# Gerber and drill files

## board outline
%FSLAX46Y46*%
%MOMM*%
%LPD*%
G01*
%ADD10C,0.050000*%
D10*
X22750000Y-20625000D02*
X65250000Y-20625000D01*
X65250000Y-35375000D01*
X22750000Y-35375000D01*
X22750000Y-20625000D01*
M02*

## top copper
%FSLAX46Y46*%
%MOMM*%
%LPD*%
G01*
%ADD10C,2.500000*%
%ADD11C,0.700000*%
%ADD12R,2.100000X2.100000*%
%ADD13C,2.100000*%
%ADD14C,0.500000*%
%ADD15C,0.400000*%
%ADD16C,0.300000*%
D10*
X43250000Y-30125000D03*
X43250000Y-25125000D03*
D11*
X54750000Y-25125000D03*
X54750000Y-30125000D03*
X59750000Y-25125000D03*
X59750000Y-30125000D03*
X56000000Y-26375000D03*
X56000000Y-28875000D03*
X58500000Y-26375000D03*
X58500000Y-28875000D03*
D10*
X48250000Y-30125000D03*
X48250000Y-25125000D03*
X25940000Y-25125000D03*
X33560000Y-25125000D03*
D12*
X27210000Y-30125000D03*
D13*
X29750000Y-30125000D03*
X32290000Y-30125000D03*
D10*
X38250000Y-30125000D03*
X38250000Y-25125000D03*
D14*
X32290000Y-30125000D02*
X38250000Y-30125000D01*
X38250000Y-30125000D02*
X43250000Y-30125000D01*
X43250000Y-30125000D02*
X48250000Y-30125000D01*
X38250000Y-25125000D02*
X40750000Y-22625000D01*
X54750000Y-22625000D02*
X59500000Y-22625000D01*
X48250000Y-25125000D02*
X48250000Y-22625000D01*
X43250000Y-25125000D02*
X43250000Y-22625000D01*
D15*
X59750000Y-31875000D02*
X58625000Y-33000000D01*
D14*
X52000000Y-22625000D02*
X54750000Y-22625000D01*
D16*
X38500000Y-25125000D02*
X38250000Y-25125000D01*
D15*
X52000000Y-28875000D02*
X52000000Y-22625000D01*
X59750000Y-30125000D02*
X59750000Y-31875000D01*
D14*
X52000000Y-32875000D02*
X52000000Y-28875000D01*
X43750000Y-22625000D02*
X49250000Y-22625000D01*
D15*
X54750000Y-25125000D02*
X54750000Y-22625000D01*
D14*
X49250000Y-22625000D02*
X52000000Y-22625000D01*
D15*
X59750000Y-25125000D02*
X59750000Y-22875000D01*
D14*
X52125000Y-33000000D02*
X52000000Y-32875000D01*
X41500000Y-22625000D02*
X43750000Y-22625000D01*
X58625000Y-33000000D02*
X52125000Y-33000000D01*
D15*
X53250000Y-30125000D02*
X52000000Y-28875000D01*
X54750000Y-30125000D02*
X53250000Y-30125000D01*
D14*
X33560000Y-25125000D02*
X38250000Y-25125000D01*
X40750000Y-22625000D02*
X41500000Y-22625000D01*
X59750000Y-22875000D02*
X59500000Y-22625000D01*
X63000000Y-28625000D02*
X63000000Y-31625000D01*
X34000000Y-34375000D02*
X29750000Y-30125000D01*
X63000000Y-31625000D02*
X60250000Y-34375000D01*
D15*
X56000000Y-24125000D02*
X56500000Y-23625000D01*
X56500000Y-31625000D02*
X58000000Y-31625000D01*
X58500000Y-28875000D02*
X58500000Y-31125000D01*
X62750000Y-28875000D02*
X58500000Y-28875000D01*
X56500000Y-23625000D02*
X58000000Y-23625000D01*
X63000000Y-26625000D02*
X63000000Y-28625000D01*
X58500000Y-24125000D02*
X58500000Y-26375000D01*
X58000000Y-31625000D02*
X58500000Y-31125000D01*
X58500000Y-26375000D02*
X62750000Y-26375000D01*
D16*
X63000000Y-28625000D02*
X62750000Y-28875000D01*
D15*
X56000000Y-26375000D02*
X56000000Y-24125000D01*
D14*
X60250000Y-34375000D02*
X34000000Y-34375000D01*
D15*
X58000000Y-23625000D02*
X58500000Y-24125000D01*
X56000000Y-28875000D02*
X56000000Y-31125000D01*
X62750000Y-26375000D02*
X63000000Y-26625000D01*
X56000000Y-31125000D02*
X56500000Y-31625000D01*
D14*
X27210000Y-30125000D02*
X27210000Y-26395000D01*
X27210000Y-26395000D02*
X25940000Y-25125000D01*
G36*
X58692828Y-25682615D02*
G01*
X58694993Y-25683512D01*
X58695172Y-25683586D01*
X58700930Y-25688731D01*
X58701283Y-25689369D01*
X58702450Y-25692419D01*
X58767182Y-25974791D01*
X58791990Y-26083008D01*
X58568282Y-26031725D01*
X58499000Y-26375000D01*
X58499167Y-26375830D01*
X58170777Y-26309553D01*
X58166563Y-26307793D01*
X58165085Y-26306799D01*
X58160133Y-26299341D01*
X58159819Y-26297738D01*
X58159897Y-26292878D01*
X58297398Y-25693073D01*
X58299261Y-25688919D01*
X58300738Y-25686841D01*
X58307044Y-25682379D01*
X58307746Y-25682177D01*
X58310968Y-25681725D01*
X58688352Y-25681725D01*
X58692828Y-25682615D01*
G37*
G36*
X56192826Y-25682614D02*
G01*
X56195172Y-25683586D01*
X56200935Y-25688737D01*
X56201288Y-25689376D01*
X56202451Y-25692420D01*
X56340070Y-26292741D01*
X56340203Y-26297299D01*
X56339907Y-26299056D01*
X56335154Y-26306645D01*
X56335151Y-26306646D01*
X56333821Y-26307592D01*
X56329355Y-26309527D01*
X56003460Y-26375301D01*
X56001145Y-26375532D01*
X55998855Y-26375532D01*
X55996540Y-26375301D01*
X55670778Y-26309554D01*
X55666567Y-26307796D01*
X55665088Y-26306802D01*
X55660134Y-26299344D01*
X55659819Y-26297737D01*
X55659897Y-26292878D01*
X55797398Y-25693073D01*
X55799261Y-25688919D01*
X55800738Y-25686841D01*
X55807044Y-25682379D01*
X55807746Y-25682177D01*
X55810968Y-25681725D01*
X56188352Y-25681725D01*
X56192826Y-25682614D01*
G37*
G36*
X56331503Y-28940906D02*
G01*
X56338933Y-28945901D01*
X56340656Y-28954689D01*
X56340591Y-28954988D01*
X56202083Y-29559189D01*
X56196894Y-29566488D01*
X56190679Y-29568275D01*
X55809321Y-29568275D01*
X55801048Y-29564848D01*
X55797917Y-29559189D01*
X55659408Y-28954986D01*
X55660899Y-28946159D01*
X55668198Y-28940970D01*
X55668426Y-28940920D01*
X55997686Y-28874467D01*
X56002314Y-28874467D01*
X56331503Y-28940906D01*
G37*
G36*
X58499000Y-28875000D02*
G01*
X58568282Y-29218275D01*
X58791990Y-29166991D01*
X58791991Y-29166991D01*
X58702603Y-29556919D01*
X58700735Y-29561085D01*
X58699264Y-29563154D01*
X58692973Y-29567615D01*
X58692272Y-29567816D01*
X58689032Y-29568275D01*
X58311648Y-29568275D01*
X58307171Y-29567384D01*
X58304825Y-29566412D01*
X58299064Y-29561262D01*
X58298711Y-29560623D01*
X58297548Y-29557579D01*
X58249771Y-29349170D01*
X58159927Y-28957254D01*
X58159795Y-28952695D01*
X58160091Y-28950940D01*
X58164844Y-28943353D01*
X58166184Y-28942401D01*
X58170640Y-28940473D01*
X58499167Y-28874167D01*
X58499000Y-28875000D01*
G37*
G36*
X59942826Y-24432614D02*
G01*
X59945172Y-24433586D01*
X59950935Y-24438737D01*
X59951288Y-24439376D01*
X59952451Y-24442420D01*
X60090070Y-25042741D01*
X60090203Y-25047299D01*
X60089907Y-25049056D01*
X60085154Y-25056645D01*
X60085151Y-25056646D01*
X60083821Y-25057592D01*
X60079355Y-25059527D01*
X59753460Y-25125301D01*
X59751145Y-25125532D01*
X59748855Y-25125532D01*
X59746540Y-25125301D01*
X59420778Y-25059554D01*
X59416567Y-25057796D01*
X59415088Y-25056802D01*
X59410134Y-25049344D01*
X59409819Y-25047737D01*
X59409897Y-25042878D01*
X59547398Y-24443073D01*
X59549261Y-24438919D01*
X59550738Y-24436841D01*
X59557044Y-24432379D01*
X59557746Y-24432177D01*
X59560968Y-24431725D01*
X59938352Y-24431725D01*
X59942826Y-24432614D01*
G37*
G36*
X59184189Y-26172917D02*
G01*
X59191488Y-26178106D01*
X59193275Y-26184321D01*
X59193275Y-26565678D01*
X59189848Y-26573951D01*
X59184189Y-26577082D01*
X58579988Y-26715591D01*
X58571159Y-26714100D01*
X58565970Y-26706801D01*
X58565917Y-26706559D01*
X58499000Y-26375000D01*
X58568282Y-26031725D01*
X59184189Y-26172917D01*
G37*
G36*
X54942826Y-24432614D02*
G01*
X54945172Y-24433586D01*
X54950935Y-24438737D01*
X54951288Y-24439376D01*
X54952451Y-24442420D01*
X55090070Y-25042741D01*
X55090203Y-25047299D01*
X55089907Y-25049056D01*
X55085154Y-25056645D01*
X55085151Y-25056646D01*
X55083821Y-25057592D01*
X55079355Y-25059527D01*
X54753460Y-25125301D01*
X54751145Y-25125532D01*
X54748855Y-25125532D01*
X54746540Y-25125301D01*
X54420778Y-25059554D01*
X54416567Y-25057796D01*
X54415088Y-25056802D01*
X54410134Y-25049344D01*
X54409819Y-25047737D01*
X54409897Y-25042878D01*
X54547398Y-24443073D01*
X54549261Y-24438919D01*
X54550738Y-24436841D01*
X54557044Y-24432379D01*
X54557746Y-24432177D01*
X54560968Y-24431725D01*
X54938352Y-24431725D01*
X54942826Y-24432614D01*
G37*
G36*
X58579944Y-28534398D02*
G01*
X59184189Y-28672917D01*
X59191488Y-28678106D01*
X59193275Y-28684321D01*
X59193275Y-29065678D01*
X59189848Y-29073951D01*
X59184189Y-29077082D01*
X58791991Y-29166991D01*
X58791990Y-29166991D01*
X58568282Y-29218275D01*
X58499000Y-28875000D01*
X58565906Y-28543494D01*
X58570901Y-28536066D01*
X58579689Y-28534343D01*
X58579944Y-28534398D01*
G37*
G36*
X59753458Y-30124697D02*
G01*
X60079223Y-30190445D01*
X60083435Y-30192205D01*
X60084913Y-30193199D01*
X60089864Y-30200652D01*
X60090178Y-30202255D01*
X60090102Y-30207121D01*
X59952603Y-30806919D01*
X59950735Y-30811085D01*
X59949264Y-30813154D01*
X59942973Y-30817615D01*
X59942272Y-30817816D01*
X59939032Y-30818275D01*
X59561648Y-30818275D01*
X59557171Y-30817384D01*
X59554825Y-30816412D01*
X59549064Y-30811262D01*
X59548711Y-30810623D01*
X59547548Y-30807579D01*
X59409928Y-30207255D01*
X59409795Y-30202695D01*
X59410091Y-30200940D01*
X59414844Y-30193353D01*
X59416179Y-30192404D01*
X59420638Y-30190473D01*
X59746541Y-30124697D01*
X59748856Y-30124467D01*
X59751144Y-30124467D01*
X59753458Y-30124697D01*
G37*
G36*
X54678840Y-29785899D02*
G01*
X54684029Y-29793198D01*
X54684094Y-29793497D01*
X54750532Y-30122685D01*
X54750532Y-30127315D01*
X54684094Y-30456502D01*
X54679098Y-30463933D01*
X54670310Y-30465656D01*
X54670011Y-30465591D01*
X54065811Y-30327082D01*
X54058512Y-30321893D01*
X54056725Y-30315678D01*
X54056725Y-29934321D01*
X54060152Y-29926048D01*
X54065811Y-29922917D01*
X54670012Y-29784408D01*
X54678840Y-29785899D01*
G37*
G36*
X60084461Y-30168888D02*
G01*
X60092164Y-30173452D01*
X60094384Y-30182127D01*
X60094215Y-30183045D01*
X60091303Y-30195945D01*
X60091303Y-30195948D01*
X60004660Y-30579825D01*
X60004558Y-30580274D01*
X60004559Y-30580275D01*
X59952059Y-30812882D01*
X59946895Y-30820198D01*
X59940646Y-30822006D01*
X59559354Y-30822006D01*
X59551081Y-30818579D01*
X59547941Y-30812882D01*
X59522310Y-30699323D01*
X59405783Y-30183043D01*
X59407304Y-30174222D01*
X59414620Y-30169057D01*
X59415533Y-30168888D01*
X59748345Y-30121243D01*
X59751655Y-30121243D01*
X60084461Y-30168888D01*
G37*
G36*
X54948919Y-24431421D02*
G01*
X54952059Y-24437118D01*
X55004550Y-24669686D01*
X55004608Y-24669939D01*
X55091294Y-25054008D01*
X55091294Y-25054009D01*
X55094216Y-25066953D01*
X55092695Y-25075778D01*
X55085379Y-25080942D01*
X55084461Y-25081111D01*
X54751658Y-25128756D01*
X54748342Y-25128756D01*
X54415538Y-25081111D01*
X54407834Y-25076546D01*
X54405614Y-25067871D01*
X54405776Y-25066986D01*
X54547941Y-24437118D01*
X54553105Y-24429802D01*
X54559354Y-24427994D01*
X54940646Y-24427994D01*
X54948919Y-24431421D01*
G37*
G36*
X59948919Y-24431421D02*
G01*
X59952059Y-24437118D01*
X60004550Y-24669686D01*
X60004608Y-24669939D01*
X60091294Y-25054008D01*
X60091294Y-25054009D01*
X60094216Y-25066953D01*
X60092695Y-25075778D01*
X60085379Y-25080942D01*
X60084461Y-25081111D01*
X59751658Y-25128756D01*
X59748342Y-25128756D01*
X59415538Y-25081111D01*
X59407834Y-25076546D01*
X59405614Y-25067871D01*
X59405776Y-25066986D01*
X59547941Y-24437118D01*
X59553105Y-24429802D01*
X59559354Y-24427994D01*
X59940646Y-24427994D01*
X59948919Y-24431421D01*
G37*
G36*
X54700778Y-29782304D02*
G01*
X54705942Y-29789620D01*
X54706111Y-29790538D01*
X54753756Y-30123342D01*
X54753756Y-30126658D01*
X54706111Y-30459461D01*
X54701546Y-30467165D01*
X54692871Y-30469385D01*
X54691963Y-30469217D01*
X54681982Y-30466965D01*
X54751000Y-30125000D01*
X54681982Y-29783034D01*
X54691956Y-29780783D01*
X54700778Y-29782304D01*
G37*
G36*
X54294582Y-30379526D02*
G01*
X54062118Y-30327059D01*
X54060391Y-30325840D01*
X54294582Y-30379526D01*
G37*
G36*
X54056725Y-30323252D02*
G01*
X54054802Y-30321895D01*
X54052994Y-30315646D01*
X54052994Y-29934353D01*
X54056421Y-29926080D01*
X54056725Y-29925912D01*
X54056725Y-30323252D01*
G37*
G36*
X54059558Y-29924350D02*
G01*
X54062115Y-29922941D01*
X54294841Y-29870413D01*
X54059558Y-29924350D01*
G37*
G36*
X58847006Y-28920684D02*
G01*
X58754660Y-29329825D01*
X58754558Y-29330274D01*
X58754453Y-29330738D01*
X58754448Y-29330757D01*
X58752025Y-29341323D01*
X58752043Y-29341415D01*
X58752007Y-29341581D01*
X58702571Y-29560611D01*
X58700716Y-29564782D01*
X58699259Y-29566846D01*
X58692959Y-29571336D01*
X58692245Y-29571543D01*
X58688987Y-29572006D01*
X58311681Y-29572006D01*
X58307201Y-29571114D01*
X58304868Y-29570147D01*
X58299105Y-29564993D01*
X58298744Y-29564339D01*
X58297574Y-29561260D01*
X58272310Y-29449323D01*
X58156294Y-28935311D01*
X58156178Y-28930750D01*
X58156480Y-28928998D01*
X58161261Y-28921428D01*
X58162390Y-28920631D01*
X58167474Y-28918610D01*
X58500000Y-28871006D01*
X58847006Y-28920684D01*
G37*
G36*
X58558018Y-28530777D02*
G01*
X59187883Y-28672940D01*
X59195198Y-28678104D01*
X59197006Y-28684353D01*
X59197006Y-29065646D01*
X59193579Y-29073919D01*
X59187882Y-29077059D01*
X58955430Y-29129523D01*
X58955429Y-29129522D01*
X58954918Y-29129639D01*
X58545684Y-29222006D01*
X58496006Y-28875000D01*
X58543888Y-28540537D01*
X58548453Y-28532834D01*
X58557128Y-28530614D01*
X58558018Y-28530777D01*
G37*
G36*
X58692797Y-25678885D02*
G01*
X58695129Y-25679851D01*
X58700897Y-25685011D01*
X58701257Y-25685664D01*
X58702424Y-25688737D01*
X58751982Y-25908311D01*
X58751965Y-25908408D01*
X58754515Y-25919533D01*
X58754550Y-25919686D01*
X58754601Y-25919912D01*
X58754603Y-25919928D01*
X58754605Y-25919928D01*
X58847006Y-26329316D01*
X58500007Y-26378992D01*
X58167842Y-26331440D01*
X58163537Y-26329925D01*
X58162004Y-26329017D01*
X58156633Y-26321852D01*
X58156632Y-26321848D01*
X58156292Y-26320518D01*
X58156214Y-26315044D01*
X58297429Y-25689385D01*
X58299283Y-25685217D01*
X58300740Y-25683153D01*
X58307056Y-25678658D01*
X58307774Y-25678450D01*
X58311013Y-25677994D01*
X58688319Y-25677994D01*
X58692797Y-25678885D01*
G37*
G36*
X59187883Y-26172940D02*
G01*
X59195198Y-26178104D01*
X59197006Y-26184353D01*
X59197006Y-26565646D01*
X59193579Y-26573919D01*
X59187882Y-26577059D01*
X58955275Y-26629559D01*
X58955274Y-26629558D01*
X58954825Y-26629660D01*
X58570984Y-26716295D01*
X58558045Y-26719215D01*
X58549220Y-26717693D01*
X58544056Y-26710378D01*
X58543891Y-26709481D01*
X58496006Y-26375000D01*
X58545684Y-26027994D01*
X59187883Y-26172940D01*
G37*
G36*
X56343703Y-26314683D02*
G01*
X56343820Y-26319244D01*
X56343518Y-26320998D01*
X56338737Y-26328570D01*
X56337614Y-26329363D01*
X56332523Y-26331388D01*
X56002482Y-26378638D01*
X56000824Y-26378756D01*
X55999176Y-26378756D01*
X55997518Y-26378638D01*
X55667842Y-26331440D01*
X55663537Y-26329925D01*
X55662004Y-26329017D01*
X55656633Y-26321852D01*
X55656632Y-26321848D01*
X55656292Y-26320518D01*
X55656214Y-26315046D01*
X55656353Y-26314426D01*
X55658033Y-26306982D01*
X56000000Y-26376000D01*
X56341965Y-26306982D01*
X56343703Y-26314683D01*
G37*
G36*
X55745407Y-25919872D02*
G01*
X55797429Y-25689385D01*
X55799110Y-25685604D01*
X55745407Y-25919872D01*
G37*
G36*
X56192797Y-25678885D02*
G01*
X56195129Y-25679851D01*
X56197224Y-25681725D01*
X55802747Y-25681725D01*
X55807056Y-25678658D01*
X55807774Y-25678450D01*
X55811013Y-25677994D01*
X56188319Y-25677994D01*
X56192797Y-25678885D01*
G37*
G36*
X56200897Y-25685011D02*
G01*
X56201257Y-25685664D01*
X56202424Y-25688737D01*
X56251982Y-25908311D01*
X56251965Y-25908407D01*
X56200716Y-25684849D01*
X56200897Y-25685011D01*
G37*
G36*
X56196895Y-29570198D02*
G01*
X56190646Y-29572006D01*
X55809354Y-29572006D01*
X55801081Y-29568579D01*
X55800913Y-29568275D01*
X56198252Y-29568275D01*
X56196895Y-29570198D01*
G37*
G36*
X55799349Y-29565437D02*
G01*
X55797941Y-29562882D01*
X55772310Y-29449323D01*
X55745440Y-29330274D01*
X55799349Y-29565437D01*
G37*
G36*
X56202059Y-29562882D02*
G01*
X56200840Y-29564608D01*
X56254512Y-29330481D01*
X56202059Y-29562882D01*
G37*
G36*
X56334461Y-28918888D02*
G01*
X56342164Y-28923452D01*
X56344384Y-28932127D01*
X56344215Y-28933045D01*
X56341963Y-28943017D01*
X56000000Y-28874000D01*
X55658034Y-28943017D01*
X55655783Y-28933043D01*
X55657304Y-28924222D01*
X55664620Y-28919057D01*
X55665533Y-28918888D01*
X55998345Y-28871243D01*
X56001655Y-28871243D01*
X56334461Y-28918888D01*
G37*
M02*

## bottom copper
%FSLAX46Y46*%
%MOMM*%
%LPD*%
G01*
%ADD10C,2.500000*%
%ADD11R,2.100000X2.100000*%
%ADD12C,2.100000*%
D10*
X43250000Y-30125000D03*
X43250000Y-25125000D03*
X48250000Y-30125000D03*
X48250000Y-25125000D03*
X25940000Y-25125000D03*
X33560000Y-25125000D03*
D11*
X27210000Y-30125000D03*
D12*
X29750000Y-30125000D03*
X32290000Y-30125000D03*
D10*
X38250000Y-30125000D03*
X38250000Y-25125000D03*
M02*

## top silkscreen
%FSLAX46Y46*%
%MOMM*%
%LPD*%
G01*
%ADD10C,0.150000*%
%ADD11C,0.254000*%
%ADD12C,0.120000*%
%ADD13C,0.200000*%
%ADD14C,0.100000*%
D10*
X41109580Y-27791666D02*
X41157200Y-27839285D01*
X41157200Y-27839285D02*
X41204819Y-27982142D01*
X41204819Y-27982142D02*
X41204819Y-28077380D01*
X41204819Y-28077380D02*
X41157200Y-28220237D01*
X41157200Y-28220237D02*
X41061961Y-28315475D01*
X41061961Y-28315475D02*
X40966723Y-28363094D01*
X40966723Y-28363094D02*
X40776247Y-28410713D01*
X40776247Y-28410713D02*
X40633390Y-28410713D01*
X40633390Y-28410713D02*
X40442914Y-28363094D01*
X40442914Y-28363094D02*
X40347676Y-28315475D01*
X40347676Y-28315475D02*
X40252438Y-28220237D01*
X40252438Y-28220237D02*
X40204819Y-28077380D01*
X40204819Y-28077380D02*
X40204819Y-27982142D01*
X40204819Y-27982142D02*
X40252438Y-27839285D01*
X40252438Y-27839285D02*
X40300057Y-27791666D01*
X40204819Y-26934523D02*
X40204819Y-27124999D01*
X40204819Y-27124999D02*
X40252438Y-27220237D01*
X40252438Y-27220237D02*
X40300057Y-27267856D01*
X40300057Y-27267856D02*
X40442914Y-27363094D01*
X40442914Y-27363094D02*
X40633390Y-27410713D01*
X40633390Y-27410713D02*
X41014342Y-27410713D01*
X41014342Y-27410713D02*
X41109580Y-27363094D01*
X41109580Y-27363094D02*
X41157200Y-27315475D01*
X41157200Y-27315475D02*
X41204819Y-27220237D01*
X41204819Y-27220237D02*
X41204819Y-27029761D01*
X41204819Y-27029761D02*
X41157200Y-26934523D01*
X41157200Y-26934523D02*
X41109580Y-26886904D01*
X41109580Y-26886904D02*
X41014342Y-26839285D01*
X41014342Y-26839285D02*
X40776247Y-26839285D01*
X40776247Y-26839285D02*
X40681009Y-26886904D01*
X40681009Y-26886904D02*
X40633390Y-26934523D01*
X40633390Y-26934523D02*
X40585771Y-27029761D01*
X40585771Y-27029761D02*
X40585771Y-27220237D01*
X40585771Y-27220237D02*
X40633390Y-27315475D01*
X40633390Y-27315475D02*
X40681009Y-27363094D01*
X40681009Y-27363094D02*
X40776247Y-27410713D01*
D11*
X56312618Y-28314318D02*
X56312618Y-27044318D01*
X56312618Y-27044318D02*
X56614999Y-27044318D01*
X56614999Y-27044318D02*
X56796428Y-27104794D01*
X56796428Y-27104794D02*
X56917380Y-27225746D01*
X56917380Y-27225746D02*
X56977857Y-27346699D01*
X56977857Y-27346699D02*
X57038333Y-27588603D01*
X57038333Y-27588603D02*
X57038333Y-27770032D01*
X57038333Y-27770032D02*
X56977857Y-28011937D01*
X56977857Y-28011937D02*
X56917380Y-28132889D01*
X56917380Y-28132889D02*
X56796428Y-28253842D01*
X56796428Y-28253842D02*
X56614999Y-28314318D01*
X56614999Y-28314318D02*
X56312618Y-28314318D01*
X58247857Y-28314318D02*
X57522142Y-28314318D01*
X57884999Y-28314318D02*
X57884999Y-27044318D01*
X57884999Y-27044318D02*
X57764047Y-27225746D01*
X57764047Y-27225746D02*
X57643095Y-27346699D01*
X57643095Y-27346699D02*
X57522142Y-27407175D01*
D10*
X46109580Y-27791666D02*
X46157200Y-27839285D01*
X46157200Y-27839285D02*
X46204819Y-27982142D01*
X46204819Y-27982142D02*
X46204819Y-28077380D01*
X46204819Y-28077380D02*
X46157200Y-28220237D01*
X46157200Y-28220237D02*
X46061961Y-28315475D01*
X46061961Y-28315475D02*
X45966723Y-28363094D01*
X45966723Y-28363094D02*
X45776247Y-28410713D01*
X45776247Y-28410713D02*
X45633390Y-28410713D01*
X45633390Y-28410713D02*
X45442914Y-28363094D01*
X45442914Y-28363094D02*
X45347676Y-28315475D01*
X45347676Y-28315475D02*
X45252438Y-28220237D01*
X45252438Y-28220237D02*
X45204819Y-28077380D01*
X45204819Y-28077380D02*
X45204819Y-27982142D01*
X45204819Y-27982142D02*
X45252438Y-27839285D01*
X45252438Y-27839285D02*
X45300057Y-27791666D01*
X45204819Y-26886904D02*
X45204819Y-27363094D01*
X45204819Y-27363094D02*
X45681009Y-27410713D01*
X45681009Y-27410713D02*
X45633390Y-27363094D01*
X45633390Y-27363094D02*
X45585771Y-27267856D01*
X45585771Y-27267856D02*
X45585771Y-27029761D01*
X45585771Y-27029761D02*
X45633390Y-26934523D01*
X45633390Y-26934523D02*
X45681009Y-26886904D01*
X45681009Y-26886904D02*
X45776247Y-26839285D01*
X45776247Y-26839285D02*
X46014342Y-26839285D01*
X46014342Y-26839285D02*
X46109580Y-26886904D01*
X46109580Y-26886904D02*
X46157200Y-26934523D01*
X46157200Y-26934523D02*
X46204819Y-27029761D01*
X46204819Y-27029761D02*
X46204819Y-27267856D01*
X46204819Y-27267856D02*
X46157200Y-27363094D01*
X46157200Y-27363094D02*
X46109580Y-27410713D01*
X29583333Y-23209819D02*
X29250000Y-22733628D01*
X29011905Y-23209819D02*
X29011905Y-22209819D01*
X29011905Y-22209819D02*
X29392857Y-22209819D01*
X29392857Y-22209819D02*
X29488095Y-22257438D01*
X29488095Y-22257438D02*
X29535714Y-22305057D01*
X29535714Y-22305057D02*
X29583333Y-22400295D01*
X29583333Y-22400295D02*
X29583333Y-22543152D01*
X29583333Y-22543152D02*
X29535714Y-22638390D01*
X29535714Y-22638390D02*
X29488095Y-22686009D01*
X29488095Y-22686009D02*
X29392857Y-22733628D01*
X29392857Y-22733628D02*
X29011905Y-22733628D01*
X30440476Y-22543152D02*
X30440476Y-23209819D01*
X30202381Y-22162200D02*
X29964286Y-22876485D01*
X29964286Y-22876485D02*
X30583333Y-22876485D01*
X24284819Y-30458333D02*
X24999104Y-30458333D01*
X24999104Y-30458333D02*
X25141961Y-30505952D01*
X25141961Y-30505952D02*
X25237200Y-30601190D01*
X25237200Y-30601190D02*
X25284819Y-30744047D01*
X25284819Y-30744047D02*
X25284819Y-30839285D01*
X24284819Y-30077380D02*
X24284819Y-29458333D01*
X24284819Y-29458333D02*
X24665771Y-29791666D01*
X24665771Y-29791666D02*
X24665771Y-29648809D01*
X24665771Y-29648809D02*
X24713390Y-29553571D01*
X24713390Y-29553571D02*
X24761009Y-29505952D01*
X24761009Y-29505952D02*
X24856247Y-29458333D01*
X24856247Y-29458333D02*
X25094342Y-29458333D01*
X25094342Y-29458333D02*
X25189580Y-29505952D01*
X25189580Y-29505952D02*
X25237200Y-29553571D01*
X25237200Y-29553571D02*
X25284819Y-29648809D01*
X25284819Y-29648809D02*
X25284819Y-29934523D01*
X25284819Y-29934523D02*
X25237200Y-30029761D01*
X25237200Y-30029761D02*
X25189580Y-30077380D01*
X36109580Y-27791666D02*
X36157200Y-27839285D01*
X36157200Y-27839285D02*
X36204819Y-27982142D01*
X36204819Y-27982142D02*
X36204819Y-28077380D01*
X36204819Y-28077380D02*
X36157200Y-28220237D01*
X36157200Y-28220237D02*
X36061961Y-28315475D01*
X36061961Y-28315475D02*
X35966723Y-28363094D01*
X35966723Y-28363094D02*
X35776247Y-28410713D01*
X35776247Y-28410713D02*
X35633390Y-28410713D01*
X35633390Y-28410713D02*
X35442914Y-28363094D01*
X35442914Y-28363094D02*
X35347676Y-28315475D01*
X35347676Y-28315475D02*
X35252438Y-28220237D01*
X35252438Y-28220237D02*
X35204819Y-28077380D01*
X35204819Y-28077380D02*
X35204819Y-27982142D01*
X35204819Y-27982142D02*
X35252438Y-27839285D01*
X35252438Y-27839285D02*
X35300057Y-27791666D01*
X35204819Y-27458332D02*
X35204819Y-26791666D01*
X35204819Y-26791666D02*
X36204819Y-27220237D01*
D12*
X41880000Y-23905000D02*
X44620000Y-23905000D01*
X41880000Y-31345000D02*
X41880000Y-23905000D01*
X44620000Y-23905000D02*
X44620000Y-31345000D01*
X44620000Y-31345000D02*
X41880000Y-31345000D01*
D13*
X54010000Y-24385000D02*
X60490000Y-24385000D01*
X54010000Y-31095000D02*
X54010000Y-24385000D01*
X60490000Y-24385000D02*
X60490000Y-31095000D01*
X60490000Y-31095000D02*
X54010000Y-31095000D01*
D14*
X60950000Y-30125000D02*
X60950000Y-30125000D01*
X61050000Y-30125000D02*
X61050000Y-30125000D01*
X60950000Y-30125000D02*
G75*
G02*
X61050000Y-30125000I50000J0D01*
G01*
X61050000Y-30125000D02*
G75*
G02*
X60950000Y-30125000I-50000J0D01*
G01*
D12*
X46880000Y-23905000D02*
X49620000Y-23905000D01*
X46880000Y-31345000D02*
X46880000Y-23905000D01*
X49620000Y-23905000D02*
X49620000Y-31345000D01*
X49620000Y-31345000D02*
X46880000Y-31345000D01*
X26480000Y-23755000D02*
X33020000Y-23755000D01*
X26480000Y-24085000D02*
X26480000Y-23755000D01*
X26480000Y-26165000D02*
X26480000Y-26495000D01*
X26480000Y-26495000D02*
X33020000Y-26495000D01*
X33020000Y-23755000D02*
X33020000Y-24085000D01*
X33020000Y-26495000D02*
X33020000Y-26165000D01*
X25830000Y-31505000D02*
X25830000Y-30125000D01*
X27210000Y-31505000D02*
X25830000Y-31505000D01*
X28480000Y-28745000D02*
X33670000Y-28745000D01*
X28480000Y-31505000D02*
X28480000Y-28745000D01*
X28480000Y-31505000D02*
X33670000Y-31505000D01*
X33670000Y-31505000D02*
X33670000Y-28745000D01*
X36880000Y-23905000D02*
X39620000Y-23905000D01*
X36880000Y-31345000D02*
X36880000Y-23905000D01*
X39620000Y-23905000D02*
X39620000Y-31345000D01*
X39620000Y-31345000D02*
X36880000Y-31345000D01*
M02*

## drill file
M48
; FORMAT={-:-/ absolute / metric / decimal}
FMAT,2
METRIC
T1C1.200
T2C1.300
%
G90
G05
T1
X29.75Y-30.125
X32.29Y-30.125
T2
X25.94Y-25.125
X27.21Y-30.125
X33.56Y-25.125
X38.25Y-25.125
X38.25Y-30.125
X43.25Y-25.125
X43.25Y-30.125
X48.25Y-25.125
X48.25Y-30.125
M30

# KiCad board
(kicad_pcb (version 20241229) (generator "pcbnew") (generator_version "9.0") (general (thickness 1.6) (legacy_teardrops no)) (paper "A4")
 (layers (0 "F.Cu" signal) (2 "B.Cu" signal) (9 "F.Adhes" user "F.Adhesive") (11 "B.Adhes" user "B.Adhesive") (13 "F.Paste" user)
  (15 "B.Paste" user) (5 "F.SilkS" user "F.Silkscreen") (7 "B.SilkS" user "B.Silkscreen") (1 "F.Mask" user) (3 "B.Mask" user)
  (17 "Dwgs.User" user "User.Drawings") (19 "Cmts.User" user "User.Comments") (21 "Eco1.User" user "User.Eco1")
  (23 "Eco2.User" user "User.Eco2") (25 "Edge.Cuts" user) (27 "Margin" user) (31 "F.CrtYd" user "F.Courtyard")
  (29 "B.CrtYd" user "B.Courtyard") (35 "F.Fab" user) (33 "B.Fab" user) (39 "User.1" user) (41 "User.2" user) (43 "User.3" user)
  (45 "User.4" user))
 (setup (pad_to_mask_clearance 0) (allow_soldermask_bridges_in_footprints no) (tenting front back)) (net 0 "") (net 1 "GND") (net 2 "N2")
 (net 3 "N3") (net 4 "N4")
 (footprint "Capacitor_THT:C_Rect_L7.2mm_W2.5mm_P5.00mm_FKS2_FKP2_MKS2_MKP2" (layer "F.Cu") (at 43.25 30.125 90)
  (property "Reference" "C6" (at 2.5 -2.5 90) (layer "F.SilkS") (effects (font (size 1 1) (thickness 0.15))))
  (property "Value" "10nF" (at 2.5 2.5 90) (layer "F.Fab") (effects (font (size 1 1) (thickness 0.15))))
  (fp_line (start 6.22 -1.37) (end 6.22 1.37) (stroke (width 0.12) (type solid)) (layer "F.SilkS"))
  (fp_line (start -1.22 -1.37) (end 6.22 -1.37) (stroke (width 0.12) (type solid)) (layer "F.SilkS"))
  (fp_line (start 6.22 1.37) (end -1.22 1.37) (stroke (width 0.12) (type solid)) (layer "F.SilkS"))
  (fp_line (start -1.22 1.37) (end -1.22 -1.37) (stroke (width 0.12) (type solid)) (layer "F.SilkS"))
  (pad "1" thru_hole circle (at 0 0 90) (size 2.5 2.5) (drill 1.3) (layers "*.Cu" "*.Mask") (remove_unused_layers no) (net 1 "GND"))
  (pad "2" thru_hole circle (at 5 0 90) (size 2.5 2.5) (drill 1.3) (layers "*.Cu" "*.Mask") (remove_unused_layers no) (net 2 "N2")))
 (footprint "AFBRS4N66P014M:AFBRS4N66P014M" (layer "F.Cu") (at 57.25 27.625)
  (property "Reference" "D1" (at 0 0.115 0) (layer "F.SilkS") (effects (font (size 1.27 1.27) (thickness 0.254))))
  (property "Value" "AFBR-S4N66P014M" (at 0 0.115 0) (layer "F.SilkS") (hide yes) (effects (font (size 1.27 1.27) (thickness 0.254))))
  (fp_line (start -3.24 -3.24) (end 3.24 -3.24) (stroke (width 0.2) (type solid)) (layer "F.SilkS"))
  (fp_line (start -3.24 3.47) (end -3.24 -3.24) (stroke (width 0.2) (type solid)) (layer "F.SilkS"))
  (fp_line (start 3.24 -3.24) (end 3.24 3.47) (stroke (width 0.2) (type solid)) (layer "F.SilkS"))
  (fp_line (start 3.24 3.47) (end -3.24 3.47) (stroke (width 0.2) (type solid)) (layer "F.SilkS"))
  (fp_line (start 3.7 2.5) (end 3.7 2.5) (stroke (width 0.1) (type solid)) (layer "F.SilkS"))
  (fp_line (start 3.8 2.5) (end 3.8 2.5) (stroke (width 0.1) (type solid)) (layer "F.SilkS"))
  (fp_arc (start 3.7 2.5) (mid 3.75 2.45) (end 3.8 2.5) (stroke (width 0.1) (type solid)) (layer "F.SilkS"))
  (fp_arc (start 3.8 2.5) (mid 3.75 2.55) (end 3.7 2.5) (stroke (width 0.1) (type solid)) (layer "F.SilkS"))
  (pad "1" smd circle (at -2.5 -2.5 90) (size 0.7 0.7) (layers "F.Cu" "F.Mask" "F.Paste") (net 2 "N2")
   (teardrops (best_length_ratio 0.5) (max_length 1) (best_width_ratio 1) (max_width 2) (curved_edges no) (filter_ratio 0.9) (enabled yes)
    (allow_two_segments yes) (prefer_zone_connections yes)))
  (pad "1" smd circle (at -2.5 2.5 90) (size 0.7 0.7) (layers "F.Cu" "F.Mask" "F.Paste") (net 2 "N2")
   (teardrops (best_length_ratio 0.5) (max_length 1) (best_width_ratio 1) (max_width 2) (curved_edges no) (filter_ratio 0.9) (enabled yes)
    (allow_two_segments yes) (prefer_zone_connections yes)))
  (pad "1" smd circle (at 2.5 -2.5 90) (size 0.7 0.7) (layers "F.Cu" "F.Mask" "F.Paste") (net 2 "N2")
   (teardrops (best_length_ratio 0.5) (max_length 1) (best_width_ratio 1) (max_width 2) (curved_edges no) (filter_ratio 0.9) (enabled yes)
    (allow_two_segments yes) (prefer_zone_connections yes)))
  (pad "1" smd circle (at 2.5 2.5 90) (size 0.7 0.7) (layers "F.Cu" "F.Mask" "F.Paste") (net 2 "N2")
   (teardrops (best_length_ratio 0.5) (max_length 1) (best_width_ratio 1) (max_width 2) (curved_edges no) (filter_ratio 0.9) (enabled yes)
    (allow_two_segments yes) (prefer_zone_connections yes)))
  (pad "2" smd circle (at -1.25 -1.25 90) (size 0.7 0.7) (layers "F.Cu" "F.Mask" "F.Paste") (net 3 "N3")
   (teardrops (best_length_ratio 0.5) (max_length 1) (best_width_ratio 1) (max_width 2) (curved_edges no) (filter_ratio 0.9) (enabled yes)
    (allow_two_segments yes) (prefer_zone_connections yes)))
  (pad "2" smd circle (at -1.25 1.25 90) (size 0.7 0.7) (layers "F.Cu" "F.Mask" "F.Paste") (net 3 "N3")
   (teardrops (best_length_ratio 0.5) (max_length 1) (best_width_ratio 1) (max_width 2) (curved_edges no) (filter_ratio 0.9) (enabled yes)
    (allow_two_segments yes) (prefer_zone_connections yes)))
  (pad "2" smd circle (at 1.25 -1.25 90) (size 0.7 0.7) (layers "F.Cu" "F.Mask" "F.Paste") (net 3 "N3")
   (teardrops (best_length_ratio 0.5) (max_length 1) (best_width_ratio 1) (max_width 2) (curved_edges no) (filter_ratio 0.9) (enabled yes)
    (allow_two_segments yes) (prefer_zone_connections yes)))
  (pad "2" smd circle (at 1.25 1.25 90) (size 0.7 0.7) (layers "F.Cu" "F.Mask" "F.Paste") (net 3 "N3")
   (teardrops (best_length_ratio 0.5) (max_length 1) (best_width_ratio 1) (max_width 2) (curved_edges no) (filter_ratio 0.9) (enabled yes)
    (allow_two_segments yes) (prefer_zone_connections yes))))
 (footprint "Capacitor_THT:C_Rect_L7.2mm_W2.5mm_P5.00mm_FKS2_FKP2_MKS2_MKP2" (layer "F.Cu") (at 48.25 30.125 90)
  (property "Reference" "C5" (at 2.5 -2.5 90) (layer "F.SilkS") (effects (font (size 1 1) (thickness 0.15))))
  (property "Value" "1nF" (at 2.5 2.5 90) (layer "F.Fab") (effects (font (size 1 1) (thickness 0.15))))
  (fp_line (start 6.22 -1.37) (end 6.22 1.37) (stroke (width 0.12) (type solid)) (layer "F.SilkS"))
  (fp_line (start -1.22 -1.37) (end 6.22 -1.37) (stroke (width 0.12) (type solid)) (layer "F.SilkS"))
  (fp_line (start 6.22 1.37) (end -1.22 1.37) (stroke (width 0.12) (type solid)) (layer "F.SilkS"))
  (fp_line (start -1.22 1.37) (end -1.22 -1.37) (stroke (width 0.12) (type solid)) (layer "F.SilkS"))
  (pad "1" thru_hole circle (at 0 0 90) (size 2.5 2.5) (drill 1.3) (layers "*.Cu" "*.Mask") (remove_unused_layers no) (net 1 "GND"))
  (pad "2" thru_hole circle (at 5 0 90) (size 2.5 2.5) (drill 1.3) (layers "*.Cu" "*.Mask") (remove_unused_layers no) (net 2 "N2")))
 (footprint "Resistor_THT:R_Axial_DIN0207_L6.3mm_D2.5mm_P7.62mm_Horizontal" (layer "F.Cu") (at 25.94 25.125)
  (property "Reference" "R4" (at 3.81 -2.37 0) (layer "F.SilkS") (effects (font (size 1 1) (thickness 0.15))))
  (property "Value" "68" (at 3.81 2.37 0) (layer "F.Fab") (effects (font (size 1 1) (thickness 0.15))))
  (fp_line (start 0.54 -1.37) (end 7.08 -1.37) (stroke (width 0.12) (type solid)) (layer "F.SilkS"))
  (fp_line (start 0.54 -1.04) (end 0.54 -1.37) (stroke (width 0.12) (type solid)) (layer "F.SilkS"))
  (fp_line (start 0.54 1.04) (end 0.54 1.37) (stroke (width 0.12) (type solid)) (layer "F.SilkS"))
  (fp_line (start 0.54 1.37) (end 7.08 1.37) (stroke (width 0.12) (type solid)) (layer "F.SilkS"))
  (fp_line (start 7.08 -1.37) (end 7.08 -1.04) (stroke (width 0.12) (type solid)) (layer "F.SilkS"))
  (fp_line (start 7.08 1.37) (end 7.08 1.04) (stroke (width 0.12) (type solid)) (layer "F.SilkS"))
  (pad "1" thru_hole circle (at 0 0) (size 2.5 2.5) (drill 1.3) (layers "*.Cu" "*.Mask") (remove_unused_layers no) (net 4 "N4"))
  (pad "2" thru_hole circle (at 7.62 0) (size 2.5 2.5) (drill 1.3) (layers "*.Cu" "*.Mask") (remove_unused_layers no) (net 2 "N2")))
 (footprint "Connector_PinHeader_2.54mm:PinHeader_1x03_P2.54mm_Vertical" (layer "F.Cu") (at 27.21 30.125 90)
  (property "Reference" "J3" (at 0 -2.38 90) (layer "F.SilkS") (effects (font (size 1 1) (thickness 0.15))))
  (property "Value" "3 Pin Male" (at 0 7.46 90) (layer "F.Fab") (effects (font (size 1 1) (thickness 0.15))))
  (fp_line (start -1.38 -1.38) (end 0 -1.38) (stroke (width 0.12) (type solid)) (layer "F.SilkS"))
  (fp_line (start -1.38 0) (end -1.38 -1.38) (stroke (width 0.12) (type solid)) (layer "F.SilkS"))
  (fp_line (start 1.38 1.27) (end 1.38 6.46) (stroke (width 0.12) (type solid)) (layer "F.SilkS"))
  (fp_line (start -1.38 1.27) (end 1.38 1.27) (stroke (width 0.12) (type solid)) (layer "F.SilkS"))
  (fp_line (start -1.38 1.27) (end -1.38 6.46) (stroke (width 0.12) (type solid)) (layer "F.SilkS"))
  (fp_line (start -1.38 6.46) (end 1.38 6.46) (stroke (width 0.12) (type solid)) (layer "F.SilkS"))
  (pad "1" thru_hole rect (at 0 0 90) (size 2.1 2.1) (drill 1.3) (layers "*.Cu" "*.Mask") (remove_unused_layers no) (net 4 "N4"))
  (pad "2" thru_hole circle (at 0 2.54 90) (size 2.1 2.1) (drill 1.2) (layers "*.Cu" "*.Mask") (remove_unused_layers no) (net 3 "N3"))
  (pad "3" thru_hole circle (at 0 5.08 90) (size 2.1 2.1) (drill 1.2) (layers "*.Cu" "*.Mask") (remove_unused_layers no) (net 1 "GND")))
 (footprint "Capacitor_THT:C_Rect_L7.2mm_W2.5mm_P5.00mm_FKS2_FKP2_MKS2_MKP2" (layer "F.Cu") (at 38.25 30.125 90)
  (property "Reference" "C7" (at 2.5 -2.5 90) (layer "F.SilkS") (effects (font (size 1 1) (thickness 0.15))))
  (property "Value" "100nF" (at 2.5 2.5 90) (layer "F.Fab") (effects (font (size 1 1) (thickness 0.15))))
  (fp_line (start 6.22 -1.37) (end 6.22 1.37) (stroke (width 0.12) (type solid)) (layer "F.SilkS"))
  (fp_line (start -1.22 -1.37) (end 6.22 -1.37) (stroke (width 0.12) (type solid)) (layer "F.SilkS"))
  (fp_line (start 6.22 1.37) (end -1.22 1.37) (stroke (width 0.12) (type solid)) (layer "F.SilkS"))
  (fp_line (start -1.22 1.37) (end -1.22 -1.37) (stroke (width 0.12) (type solid)) (layer "F.SilkS"))
  (pad "1" thru_hole circle (at 0 0 90) (size 2.5 2.5) (drill 1.3) (layers "*.Cu" "*.Mask") (remove_unused_layers no) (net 1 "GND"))
  (pad "2" thru_hole circle (at 5 0 90) (size 2.5 2.5) (drill 1.3) (layers "*.Cu" "*.Mask") (remove_unused_layers no) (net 2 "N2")))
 (gr_rect (start 22.75 20.625) (end 65.25 35.375) (stroke (width 0.05) (type default)) (fill no) (layer "Edge.Cuts"))
 (segment (start 32.29 30.125) (end 38.25 30.125) (width 0.5) (layer "F.Cu") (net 1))
 (segment (start 38.25 30.125) (end 43.25 30.125) (width 0.5) (layer "F.Cu") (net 1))
 (segment (start 43.25 30.125) (end 48.25 30.125) (width 0.5) (layer "F.Cu") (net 1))
 (segment (start 38.25 25.125) (end 40.75 22.625) (width 0.5) (layer "F.Cu") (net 2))
 (segment (start 54.75 22.625) (end 59.5 22.625) (width 0.5) (layer "F.Cu") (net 2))
 (segment (start 48.25 25.125) (end 48.25 22.625) (width 0.5) (layer "F.Cu") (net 2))
 (segment (start 43.25 25.125) (end 43.25 22.625) (width 0.5) (layer "F.Cu") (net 2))
 (segment (start 59.75 31.875) (end 58.625 33) (width 0.4) (layer "F.Cu") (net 2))
 (segment (start 52 22.625) (end 54.75 22.625) (width 0.5) (layer "F.Cu") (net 2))
 (segment (start 38.5 25.125) (end 38.25 25.125) (width 0.3) (layer "F.Cu") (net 2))
 (segment (start 52 28.875) (end 52 22.625) (width 0.4) (layer "F.Cu") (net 2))
 (segment (start 59.75 30.125) (end 59.75 31.875) (width 0.4) (layer "F.Cu") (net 2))
 (segment (start 52 32.875) (end 52 28.875) (width 0.5) (layer "F.Cu") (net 2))
 (segment (start 43.75 22.625) (end 49.25 22.625) (width 0.5) (layer "F.Cu") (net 2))
 (segment (start 54.75 25.125) (end 54.75 22.625) (width 0.4) (layer "F.Cu") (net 2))
 (segment (start 49.25 22.625) (end 52 22.625) (width 0.5) (layer "F.Cu") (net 2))
 (segment (start 59.75 25.125) (end 59.75 22.875) (width 0.4) (layer "F.Cu") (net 2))
 (segment (start 52.125 33) (end 52 32.875) (width 0.5) (layer "F.Cu") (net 2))
 (segment (start 41.5 22.625) (end 43.75 22.625) (width 0.5) (layer "F.Cu") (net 2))
 (segment (start 58.625 33) (end 52.125 33) (width 0.5) (layer "F.Cu") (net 2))
 (segment (start 53.25 30.125) (end 52 28.875) (width 0.4) (layer "F.Cu") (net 2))
 (segment (start 54.75 30.125) (end 53.25 30.125) (width 0.4) (layer "F.Cu") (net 2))
 (segment (start 33.56 25.125) (end 38.25 25.125) (width 0.5) (layer "F.Cu") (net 2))
 (segment (start 40.75 22.625) (end 41.5 22.625) (width 0.5) (layer "F.Cu") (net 2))
 (segment (start 59.75 22.875) (end 59.5 22.625) (width 0.5) (layer "F.Cu") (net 2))
 (segment (start 63 28.625) (end 63 31.625) (width 0.5) (layer "F.Cu") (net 3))
 (segment (start 34 34.375) (end 29.75 30.125) (width 0.5) (layer "F.Cu") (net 3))
 (segment (start 63 31.625) (end 60.25 34.375) (width 0.5) (layer "F.Cu") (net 3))
 (segment (start 56 24.125) (end 56.5 23.625) (width 0.4) (layer "F.Cu") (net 3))
 (segment (start 56.5 31.625) (end 58 31.625) (width 0.4) (layer "F.Cu") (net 3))
 (segment (start 58.5 28.875) (end 58.5 31.125) (width 0.4) (layer "F.Cu") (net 3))
 (segment (start 62.75 28.875) (end 58.5 28.875) (width 0.4) (layer "F.Cu") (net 3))
 (segment (start 56.5 23.625) (end 58 23.625) (width 0.4) (layer "F.Cu") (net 3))
 (segment (start 63 26.625) (end 63 28.625) (width 0.4) (layer "F.Cu") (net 3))
 (segment (start 58.5 24.125) (end 58.5 26.375) (width 0.4) (layer "F.Cu") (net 3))
 (segment (start 58 31.625) (end 58.5 31.125) (width 0.4) (layer "F.Cu") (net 3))
 (segment (start 58.5 26.375) (end 62.75 26.375) (width 0.4) (layer "F.Cu") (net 3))
 (segment (start 63 28.625) (end 62.75 28.875) (width 0.3) (layer "F.Cu") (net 3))
 (segment (start 56 26.375) (end 56 24.125) (width 0.4) (layer "F.Cu") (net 3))
 (segment (start 60.25 34.375) (end 34 34.375) (width 0.5) (layer "F.Cu") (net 3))
 (segment (start 58 23.625) (end 58.5 24.125) (width 0.4) (layer "F.Cu") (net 3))
 (segment (start 56 28.875) (end 56 31.125) (width 0.4) (layer "F.Cu") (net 3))
 (segment (start 62.75 26.375) (end 63 26.625) (width 0.4) (layer "F.Cu") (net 3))
 (segment (start 56 31.125) (end 56.5 31.625) (width 0.4) (layer "F.Cu") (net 3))
 (segment (start 27.21 30.125) (end 27.21 26.395) (width 0.5) (layer "F.Cu") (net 4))
 (segment (start 27.21 26.395) (end 25.94 25.125) (width 0.5) (layer "F.Cu") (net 4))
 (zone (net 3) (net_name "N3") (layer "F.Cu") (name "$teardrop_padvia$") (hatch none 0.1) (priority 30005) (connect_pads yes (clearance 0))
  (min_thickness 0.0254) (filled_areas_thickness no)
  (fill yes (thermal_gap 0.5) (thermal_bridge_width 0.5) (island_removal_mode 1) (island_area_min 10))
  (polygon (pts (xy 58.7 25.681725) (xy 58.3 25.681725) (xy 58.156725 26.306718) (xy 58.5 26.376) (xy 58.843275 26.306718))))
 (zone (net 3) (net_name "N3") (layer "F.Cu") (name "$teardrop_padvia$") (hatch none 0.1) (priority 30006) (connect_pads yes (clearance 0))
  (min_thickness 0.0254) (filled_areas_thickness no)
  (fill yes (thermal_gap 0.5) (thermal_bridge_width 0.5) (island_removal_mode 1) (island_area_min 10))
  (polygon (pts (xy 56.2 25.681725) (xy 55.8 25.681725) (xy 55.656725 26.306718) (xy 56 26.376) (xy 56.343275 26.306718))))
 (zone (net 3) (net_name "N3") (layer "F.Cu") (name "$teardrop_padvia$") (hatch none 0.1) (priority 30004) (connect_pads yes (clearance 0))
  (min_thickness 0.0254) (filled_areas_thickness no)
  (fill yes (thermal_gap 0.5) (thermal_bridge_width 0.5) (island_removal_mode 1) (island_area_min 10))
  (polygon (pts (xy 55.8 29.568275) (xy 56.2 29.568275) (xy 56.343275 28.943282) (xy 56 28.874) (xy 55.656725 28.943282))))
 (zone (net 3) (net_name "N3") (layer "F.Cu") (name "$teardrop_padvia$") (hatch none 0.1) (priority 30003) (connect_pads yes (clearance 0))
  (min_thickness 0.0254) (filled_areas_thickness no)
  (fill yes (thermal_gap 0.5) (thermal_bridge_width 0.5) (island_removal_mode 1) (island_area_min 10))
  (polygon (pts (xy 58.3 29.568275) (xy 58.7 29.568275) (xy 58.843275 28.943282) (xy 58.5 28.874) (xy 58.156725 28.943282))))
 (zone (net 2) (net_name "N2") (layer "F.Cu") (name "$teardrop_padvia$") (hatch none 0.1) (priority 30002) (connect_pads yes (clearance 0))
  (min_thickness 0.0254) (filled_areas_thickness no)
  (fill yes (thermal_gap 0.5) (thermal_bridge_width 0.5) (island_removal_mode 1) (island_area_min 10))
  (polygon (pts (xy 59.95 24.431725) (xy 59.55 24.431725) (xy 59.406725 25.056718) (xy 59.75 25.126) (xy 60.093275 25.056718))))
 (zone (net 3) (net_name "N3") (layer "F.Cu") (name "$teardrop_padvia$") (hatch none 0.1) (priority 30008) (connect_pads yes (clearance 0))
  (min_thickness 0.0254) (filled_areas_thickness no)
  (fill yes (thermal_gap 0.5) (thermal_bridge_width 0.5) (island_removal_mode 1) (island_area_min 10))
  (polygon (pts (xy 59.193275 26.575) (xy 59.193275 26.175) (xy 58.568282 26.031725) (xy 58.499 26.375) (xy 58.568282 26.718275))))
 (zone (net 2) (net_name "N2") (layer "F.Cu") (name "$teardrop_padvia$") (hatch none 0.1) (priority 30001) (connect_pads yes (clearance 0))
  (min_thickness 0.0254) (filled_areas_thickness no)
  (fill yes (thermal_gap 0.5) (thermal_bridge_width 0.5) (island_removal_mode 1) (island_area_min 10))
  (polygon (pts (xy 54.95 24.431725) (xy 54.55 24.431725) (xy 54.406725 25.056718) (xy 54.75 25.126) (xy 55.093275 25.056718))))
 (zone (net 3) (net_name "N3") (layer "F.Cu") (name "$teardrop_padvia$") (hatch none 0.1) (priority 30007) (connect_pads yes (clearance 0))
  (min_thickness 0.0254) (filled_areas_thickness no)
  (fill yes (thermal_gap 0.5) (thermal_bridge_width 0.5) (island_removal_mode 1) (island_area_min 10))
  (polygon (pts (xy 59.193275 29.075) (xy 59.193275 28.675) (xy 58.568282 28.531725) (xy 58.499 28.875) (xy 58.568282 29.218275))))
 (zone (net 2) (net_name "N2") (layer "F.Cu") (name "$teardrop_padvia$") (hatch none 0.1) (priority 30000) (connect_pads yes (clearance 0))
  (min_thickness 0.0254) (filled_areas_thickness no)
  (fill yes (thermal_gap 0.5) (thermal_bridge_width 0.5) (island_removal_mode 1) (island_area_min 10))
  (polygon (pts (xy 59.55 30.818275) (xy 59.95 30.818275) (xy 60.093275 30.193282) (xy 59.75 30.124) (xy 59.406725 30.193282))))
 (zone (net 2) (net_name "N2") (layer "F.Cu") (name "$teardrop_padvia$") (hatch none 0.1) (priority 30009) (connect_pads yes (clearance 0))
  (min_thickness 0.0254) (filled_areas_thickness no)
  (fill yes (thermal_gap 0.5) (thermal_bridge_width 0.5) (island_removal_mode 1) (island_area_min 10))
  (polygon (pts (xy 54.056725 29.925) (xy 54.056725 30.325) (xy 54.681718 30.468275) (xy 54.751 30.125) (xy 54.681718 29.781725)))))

